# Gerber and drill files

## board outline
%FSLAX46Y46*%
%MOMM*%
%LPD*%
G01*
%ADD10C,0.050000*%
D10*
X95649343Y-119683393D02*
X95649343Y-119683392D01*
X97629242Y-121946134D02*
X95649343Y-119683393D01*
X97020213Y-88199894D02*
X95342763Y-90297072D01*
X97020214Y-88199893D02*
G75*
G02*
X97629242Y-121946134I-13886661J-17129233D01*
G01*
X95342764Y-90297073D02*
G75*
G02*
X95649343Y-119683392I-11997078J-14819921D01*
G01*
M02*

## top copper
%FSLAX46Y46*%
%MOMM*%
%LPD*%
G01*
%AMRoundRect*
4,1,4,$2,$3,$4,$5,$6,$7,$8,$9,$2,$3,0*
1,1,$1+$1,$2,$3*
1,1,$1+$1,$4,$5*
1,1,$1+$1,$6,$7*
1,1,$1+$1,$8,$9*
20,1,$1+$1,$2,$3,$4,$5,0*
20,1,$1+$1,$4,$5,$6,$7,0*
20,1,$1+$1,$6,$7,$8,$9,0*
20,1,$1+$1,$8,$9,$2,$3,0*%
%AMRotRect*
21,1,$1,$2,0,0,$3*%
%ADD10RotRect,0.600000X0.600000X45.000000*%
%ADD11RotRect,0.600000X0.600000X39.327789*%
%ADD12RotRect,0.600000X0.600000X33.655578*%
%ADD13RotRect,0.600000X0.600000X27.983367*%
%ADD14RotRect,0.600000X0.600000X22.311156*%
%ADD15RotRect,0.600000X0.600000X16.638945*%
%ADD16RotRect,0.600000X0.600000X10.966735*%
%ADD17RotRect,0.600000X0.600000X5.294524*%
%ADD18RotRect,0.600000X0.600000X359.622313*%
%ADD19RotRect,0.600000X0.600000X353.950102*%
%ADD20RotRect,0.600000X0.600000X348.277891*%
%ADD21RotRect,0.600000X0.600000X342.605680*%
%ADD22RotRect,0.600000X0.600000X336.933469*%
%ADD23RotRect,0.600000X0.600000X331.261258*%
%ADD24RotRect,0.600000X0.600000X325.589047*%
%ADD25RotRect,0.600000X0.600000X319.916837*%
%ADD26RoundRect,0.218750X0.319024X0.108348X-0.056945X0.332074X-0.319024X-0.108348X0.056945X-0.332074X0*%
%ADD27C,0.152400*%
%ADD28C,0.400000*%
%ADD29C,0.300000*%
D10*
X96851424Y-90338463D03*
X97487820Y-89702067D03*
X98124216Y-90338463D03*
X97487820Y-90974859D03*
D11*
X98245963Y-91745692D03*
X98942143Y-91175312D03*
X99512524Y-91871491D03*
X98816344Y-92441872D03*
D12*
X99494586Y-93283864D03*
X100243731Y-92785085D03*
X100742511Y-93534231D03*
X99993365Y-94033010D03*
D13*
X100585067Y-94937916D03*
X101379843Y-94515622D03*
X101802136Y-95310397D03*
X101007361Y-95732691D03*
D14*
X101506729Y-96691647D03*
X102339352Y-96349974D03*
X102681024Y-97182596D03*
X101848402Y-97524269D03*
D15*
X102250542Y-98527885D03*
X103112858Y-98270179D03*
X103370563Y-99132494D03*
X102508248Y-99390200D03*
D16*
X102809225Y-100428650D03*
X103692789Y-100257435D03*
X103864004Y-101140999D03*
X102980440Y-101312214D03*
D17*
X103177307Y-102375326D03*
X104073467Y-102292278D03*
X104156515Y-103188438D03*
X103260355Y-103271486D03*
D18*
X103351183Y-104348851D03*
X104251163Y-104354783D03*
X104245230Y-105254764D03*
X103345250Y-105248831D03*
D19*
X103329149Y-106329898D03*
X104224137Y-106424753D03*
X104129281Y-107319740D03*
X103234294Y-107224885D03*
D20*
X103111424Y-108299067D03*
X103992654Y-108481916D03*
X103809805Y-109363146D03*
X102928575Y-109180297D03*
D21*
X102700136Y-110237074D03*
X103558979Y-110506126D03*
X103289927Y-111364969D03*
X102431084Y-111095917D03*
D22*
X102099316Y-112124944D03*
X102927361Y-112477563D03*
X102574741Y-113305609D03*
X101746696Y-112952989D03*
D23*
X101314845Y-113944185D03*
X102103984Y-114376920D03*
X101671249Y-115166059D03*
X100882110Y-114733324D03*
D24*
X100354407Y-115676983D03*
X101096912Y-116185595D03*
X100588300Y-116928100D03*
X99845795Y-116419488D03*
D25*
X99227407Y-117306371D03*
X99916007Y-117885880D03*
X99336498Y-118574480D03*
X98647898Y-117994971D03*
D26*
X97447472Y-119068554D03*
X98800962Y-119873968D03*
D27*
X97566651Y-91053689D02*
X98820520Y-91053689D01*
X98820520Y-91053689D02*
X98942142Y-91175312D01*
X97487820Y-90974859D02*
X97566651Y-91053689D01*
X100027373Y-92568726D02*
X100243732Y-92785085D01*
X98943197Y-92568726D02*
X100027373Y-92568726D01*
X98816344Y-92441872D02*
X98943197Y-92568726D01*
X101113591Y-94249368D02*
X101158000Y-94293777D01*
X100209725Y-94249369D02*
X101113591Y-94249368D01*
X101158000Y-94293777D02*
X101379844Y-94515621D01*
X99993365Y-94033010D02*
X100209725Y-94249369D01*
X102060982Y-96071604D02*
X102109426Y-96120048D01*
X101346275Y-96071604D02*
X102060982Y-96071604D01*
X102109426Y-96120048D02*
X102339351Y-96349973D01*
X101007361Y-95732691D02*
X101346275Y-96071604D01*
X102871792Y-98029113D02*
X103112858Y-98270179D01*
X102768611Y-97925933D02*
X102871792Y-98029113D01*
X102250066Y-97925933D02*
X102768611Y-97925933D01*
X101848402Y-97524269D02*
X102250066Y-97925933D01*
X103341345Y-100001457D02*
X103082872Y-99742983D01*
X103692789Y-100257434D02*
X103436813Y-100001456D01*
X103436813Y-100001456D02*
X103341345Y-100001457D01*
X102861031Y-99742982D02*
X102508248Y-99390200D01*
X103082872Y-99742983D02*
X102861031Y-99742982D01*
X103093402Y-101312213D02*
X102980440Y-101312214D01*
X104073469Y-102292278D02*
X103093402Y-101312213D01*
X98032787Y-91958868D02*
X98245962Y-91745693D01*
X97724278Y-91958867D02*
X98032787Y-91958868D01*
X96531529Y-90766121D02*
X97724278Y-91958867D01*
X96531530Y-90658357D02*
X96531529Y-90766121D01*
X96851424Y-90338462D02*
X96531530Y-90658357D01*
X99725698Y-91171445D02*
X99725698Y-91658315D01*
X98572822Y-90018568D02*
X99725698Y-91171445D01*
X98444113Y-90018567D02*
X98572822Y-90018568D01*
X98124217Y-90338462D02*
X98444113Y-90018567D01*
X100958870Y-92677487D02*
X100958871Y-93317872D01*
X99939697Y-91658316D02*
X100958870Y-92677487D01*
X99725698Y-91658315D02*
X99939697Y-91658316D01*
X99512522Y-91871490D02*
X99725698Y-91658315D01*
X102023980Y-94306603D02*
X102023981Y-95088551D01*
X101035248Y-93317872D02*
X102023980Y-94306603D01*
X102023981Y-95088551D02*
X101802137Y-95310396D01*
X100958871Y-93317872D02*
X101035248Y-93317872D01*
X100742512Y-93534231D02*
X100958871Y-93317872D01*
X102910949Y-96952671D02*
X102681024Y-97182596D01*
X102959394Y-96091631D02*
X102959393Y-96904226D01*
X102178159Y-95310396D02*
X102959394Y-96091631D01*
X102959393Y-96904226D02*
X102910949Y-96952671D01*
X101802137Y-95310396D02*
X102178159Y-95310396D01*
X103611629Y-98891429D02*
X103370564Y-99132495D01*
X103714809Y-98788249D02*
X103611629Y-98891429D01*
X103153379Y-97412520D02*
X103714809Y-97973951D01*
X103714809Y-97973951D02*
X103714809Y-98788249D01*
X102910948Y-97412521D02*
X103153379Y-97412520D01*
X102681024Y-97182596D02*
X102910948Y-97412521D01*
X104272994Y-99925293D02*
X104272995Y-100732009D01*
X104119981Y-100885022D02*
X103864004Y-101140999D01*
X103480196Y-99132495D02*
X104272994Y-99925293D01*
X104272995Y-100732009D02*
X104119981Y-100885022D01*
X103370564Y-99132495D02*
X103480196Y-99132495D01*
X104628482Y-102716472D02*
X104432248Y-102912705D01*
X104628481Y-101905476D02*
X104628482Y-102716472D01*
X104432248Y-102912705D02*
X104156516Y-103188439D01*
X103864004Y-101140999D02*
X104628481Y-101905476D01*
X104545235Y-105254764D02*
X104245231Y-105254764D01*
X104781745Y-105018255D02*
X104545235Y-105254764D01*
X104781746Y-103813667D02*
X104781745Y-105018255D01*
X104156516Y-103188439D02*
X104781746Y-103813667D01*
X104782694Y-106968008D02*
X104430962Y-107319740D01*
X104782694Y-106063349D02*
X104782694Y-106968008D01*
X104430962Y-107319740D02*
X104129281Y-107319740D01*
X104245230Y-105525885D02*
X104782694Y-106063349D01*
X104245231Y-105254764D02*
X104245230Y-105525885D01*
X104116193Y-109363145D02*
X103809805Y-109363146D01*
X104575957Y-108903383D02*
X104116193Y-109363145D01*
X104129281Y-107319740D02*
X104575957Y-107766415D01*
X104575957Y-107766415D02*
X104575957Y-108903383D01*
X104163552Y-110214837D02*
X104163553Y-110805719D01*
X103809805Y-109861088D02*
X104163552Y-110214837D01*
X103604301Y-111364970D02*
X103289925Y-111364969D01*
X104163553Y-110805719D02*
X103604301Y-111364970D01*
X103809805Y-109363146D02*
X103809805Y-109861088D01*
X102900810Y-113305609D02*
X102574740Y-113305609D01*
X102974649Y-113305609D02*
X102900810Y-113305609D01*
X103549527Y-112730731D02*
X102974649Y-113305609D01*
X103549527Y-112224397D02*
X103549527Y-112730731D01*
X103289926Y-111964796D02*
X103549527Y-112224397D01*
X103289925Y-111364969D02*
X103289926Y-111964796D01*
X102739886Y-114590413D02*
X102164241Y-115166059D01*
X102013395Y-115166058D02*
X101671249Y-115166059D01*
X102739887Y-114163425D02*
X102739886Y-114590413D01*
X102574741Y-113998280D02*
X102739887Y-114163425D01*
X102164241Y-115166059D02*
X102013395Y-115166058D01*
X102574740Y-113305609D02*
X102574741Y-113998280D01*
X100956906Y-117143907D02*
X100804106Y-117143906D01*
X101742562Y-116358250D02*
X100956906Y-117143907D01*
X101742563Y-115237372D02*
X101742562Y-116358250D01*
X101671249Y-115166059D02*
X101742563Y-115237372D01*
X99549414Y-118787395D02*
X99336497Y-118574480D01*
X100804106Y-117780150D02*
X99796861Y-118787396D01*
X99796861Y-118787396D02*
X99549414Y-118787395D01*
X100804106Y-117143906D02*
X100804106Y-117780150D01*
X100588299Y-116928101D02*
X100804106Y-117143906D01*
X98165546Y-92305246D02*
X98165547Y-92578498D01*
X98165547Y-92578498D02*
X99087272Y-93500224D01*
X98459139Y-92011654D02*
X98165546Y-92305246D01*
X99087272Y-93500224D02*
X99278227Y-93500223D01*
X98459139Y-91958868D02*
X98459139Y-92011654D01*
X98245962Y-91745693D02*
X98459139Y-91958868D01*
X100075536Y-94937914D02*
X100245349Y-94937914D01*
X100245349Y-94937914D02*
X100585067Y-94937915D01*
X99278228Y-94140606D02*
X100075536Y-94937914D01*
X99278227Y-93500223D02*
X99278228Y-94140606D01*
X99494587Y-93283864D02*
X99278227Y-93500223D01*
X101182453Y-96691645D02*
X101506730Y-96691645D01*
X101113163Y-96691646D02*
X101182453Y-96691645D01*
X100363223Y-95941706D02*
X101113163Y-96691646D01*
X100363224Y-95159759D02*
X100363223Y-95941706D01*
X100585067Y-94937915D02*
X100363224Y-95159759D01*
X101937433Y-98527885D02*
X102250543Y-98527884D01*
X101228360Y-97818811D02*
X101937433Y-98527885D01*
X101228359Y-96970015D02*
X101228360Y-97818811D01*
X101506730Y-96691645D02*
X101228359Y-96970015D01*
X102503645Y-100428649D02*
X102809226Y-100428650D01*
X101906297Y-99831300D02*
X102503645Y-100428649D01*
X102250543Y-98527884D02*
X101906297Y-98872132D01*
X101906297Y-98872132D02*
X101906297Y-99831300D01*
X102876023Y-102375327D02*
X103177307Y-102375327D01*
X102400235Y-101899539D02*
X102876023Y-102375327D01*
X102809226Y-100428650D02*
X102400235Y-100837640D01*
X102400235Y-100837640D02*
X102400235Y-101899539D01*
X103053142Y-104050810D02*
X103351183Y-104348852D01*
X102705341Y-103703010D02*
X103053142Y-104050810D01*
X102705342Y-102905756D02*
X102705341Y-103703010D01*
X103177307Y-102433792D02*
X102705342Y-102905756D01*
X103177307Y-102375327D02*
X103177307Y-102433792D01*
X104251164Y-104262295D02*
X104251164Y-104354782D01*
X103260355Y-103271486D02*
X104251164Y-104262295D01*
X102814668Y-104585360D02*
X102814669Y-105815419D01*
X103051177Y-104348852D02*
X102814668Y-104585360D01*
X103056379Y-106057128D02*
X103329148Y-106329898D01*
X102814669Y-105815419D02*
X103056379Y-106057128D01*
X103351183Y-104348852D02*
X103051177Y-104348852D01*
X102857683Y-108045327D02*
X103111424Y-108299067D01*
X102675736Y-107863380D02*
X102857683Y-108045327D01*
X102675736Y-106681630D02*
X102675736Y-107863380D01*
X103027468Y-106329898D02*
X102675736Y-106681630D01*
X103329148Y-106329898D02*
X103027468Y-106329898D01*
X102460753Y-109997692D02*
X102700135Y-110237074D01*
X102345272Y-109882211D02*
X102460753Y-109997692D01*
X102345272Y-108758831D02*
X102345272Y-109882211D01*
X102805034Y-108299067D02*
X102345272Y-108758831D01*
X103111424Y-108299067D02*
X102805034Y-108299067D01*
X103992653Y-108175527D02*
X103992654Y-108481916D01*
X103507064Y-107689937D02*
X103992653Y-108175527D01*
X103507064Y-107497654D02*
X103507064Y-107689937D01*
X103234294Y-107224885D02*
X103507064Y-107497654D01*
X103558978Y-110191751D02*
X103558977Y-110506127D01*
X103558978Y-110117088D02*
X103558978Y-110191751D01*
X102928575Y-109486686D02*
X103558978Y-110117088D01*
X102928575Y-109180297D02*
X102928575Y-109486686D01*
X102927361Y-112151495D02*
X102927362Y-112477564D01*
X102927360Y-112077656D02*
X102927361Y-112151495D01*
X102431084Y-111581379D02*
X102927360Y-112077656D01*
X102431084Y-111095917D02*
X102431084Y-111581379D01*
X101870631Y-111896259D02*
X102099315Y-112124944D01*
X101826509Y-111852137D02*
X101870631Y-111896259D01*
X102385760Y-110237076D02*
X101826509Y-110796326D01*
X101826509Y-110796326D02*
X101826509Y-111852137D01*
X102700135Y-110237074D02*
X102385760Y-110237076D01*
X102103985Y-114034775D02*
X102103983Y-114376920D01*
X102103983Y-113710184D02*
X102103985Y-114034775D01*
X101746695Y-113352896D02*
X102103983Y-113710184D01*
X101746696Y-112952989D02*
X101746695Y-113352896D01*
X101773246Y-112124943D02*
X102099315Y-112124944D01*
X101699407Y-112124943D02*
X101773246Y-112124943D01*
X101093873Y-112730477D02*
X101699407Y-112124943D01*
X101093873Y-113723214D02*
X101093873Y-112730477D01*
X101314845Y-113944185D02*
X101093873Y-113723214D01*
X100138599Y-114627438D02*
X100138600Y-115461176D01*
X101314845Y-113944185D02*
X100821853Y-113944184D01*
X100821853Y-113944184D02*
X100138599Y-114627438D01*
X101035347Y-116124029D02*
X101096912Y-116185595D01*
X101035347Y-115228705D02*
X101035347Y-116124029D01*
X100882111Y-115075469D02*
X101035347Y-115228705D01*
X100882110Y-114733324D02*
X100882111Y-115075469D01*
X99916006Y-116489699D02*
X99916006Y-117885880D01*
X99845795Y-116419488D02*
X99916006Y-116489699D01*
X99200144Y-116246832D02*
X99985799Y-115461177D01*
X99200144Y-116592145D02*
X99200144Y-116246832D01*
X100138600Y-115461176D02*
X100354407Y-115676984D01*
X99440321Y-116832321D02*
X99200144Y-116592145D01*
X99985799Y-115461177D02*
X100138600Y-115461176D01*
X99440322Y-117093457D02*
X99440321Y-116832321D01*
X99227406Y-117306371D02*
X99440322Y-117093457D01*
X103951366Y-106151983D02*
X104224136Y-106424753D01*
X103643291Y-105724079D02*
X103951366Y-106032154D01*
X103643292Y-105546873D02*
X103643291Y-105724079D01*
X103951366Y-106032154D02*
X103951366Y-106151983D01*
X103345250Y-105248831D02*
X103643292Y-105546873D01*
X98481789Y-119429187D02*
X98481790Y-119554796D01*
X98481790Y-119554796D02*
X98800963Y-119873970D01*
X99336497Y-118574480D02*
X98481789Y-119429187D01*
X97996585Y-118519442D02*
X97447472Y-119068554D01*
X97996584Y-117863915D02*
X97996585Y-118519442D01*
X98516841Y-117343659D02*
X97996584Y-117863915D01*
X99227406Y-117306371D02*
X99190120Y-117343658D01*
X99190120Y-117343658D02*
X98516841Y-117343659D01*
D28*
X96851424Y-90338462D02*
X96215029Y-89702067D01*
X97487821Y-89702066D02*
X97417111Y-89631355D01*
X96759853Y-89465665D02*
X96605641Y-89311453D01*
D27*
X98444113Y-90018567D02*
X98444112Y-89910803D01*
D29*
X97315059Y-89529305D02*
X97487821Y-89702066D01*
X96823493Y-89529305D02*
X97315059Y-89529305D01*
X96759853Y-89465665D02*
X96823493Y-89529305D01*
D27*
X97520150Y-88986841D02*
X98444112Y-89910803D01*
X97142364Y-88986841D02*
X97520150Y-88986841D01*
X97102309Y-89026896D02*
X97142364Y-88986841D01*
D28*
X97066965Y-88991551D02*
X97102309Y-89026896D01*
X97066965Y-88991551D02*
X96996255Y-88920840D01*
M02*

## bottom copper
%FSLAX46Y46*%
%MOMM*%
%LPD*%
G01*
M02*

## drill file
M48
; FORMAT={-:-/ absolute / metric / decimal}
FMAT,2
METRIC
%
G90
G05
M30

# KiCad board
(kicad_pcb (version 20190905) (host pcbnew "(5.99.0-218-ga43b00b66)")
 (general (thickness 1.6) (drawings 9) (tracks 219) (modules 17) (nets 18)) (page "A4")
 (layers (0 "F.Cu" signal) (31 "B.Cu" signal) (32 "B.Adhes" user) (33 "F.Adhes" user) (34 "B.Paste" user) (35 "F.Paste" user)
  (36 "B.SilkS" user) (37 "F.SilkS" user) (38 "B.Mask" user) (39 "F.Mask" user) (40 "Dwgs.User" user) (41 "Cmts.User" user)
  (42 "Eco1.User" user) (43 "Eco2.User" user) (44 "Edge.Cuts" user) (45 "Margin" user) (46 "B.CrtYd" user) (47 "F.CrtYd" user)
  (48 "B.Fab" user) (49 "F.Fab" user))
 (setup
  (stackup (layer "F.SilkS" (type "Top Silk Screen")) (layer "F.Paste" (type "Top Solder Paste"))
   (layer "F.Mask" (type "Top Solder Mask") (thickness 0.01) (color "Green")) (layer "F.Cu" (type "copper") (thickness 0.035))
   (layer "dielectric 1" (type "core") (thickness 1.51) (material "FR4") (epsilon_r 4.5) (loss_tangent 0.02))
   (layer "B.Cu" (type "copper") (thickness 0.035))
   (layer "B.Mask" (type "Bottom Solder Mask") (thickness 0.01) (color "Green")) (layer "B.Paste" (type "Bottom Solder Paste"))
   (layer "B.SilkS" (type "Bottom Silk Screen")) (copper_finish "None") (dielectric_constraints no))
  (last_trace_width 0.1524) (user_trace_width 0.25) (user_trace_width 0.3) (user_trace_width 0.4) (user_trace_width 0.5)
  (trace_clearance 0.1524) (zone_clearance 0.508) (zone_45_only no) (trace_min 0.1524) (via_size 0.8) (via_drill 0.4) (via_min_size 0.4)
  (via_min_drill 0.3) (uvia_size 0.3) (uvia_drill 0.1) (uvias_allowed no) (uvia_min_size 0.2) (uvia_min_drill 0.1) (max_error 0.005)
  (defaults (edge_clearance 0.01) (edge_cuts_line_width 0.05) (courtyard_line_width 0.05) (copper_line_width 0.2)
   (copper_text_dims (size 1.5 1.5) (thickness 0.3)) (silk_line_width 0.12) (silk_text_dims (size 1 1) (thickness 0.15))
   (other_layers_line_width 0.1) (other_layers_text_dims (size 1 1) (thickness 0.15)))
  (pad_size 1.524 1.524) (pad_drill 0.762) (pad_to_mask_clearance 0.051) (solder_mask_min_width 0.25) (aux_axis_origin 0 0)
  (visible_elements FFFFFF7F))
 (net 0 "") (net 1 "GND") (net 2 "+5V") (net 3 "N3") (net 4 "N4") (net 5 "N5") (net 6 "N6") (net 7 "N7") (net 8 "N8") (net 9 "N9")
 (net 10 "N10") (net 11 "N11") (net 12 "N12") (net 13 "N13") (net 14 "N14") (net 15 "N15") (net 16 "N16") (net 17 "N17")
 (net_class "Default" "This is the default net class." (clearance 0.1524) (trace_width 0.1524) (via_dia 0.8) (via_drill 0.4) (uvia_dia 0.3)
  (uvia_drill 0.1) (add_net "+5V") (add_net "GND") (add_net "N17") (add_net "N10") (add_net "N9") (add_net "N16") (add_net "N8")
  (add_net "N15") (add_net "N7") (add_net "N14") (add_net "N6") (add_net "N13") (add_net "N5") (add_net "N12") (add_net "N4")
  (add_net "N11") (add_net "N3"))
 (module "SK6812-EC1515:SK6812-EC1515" (layer "F.Cu") (at 97.48782 90.974859 45)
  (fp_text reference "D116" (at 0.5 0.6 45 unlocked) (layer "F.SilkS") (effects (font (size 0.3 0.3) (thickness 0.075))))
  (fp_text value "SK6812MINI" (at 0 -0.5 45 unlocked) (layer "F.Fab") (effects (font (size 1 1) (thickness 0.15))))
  (pad "4" smd rect (at 0 -0.9 45) (size 0.6 0.6) (layers "F.Cu" "F.Paste" "F.Mask") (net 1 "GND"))
  (pad "3" smd rect (at 0.9 -0.9 45) (size 0.6 0.6) (layers "F.Cu" "F.Paste" "F.Mask"))
  (pad "2" smd rect (at 0.9 0 45) (size 0.6 0.6) (layers "F.Cu" "F.Paste" "F.Mask") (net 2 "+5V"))
  (pad "1" smd rect (at 0 0 45) (size 0.6 0.6) (layers "F.Cu" "F.Paste" "F.Mask") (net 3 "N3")))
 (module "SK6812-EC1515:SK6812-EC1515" (layer "F.Cu") (at 98.816344 92.441872 39.32778911)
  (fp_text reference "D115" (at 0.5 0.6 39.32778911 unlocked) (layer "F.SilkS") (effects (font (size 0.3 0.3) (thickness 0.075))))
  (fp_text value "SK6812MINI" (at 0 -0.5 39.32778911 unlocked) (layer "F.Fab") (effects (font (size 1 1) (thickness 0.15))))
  (pad "4" smd rect (at 0 -0.9 39.3277891) (size 0.6 0.6) (layers "F.Cu" "F.Paste" "F.Mask") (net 1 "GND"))
  (pad "3" smd rect (at 0.9 -0.9 39.3277891) (size 0.6 0.6) (layers "F.Cu" "F.Paste" "F.Mask") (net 3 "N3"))
  (pad "2" smd rect (at 0.9 0 39.3277891) (size 0.6 0.6) (layers "F.Cu" "F.Paste" "F.Mask") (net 2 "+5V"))
  (pad "1" smd rect (at 0 0 39.3277891) (size 0.6 0.6) (layers "F.Cu" "F.Paste" "F.Mask") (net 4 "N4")))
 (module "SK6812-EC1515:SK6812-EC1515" (layer "F.Cu") (at 99.993365 94.03301 33.65557821)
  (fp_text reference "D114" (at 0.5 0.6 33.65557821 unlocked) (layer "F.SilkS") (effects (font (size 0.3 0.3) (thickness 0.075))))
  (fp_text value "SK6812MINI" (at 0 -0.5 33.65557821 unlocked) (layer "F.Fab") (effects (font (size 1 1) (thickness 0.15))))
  (pad "4" smd rect (at 0 -0.9 33.6555782) (size 0.6 0.6) (layers "F.Cu" "F.Paste" "F.Mask") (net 1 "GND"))
  (pad "3" smd rect (at 0.9 -0.9 33.6555782) (size 0.6 0.6) (layers "F.Cu" "F.Paste" "F.Mask") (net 4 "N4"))
  (pad "2" smd rect (at 0.9 0 33.6555782) (size 0.6 0.6) (layers "F.Cu" "F.Paste" "F.Mask") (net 2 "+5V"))
  (pad "1" smd rect (at 0 0 33.6555782) (size 0.6 0.6) (layers "F.Cu" "F.Paste" "F.Mask") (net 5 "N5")))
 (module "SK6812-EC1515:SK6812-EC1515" (layer "F.Cu") (at 101.007361 95.732691 27.98336732)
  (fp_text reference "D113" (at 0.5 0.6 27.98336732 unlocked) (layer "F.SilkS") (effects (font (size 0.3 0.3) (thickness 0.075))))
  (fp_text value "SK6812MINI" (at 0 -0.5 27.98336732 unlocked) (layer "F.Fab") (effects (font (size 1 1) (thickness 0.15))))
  (pad "4" smd rect (at 0 -0.9 27.9833673) (size 0.6 0.6) (layers "F.Cu" "F.Paste" "F.Mask") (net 1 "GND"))
  (pad "3" smd rect (at 0.9 -0.9 27.9833673) (size 0.6 0.6) (layers "F.Cu" "F.Paste" "F.Mask") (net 5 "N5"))
  (pad "2" smd rect (at 0.9 0 27.9833673) (size 0.6 0.6) (layers "F.Cu" "F.Paste" "F.Mask") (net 2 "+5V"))
  (pad "1" smd rect (at 0 0 27.9833673) (size 0.6 0.6) (layers "F.Cu" "F.Paste" "F.Mask") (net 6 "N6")))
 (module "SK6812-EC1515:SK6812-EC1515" (layer "F.Cu") (at 101.848402 97.524269 22.31115642)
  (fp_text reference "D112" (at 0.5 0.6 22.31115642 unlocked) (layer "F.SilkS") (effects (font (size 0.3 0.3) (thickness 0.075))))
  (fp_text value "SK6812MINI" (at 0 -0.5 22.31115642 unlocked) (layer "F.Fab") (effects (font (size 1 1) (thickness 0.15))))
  (pad "4" smd rect (at 0 -0.9 22.3111564) (size 0.6 0.6) (layers "F.Cu" "F.Paste" "F.Mask") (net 1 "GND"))
  (pad "3" smd rect (at 0.9 -0.9 22.3111564) (size 0.6 0.6) (layers "F.Cu" "F.Paste" "F.Mask") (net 6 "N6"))
  (pad "2" smd rect (at 0.9 0 22.3111564) (size 0.6 0.6) (layers "F.Cu" "F.Paste" "F.Mask") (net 2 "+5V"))
  (pad "1" smd rect (at 0 0 22.3111564) (size 0.6 0.6) (layers "F.Cu" "F.Paste" "F.Mask") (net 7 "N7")))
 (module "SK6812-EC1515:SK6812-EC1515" (layer "F.Cu") (at 102.508248 99.3902 16.63894553)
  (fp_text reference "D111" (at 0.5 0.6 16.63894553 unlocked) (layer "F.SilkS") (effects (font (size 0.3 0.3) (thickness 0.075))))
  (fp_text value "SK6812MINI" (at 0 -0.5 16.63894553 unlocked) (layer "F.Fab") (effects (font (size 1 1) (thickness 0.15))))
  (pad "4" smd rect (at 0 -0.9 16.6389455) (size 0.6 0.6) (layers "F.Cu" "F.Paste" "F.Mask") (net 1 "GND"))
  (pad "3" smd rect (at 0.9 -0.9 16.6389455) (size 0.6 0.6) (layers "F.Cu" "F.Paste" "F.Mask") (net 7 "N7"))
  (pad "2" smd rect (at 0.9 0 16.6389455) (size 0.6 0.6) (layers "F.Cu" "F.Paste" "F.Mask") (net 2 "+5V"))
  (pad "1" smd rect (at 0 0 16.6389455) (size 0.6 0.6) (layers "F.Cu" "F.Paste" "F.Mask") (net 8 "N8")))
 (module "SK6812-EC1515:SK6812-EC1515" (layer "F.Cu") (at 102.98044 101.312214 10.96673463)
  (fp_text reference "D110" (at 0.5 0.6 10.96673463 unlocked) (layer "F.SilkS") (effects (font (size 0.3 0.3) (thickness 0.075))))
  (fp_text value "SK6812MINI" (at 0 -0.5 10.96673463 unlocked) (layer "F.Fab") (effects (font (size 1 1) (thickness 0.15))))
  (pad "4" smd rect (at 0 -0.9 10.9667346) (size 0.6 0.6) (layers "F.Cu" "F.Paste" "F.Mask") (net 1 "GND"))
  (pad "3" smd rect (at 0.9 -0.9 10.9667346) (size 0.6 0.6) (layers "F.Cu" "F.Paste" "F.Mask") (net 8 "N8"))
  (pad "2" smd rect (at 0.9 0 10.9667346) (size 0.6 0.6) (layers "F.Cu" "F.Paste" "F.Mask") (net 2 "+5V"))
  (pad "1" smd rect (at 0 0 10.9667346) (size 0.6 0.6) (layers "F.Cu" "F.Paste" "F.Mask") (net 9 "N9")))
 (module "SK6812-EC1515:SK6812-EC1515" (layer "F.Cu") (at 103.260355 103.271486 5.29452374)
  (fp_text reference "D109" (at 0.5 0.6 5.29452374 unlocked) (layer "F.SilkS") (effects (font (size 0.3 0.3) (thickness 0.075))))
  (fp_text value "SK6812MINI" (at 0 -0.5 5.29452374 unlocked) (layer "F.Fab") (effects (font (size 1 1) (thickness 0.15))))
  (pad "4" smd rect (at 0 -0.9 5.2945237) (size 0.6 0.6) (layers "F.Cu" "F.Paste" "F.Mask") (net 1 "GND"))
  (pad "3" smd rect (at 0.9 -0.9 5.2945237) (size 0.6 0.6) (layers "F.Cu" "F.Paste" "F.Mask") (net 9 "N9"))
  (pad "2" smd rect (at 0.9 0 5.2945237) (size 0.6 0.6) (layers "F.Cu" "F.Paste" "F.Mask") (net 2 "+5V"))
  (pad "1" smd rect (at 0 0 5.2945237) (size 0.6 0.6) (layers "F.Cu" "F.Paste" "F.Mask") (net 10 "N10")))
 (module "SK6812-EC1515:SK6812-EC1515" (layer "F.Cu") (at 103.34525 105.248831 -0.37768716)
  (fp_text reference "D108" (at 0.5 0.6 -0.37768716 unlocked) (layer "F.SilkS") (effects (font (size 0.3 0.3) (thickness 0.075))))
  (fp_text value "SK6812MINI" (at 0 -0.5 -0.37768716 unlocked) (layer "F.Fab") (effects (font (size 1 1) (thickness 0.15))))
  (pad "4" smd rect (at 0 -0.9 359.6223128) (size 0.6 0.6) (layers "F.Cu" "F.Paste" "F.Mask") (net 1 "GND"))
  (pad "3" smd rect (at 0.9 -0.9 359.6223128) (size 0.6 0.6) (layers "F.Cu" "F.Paste" "F.Mask") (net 10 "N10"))
  (pad "2" smd rect (at 0.9 0 359.6223128) (size 0.6 0.6) (layers "F.Cu" "F.Paste" "F.Mask") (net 2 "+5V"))
  (pad "1" smd rect (at 0 0 359.6223128) (size 0.6 0.6) (layers "F.Cu" "F.Paste" "F.Mask") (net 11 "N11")))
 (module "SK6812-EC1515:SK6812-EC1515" (layer "F.Cu") (at 103.234294 107.224885 -6.04989805)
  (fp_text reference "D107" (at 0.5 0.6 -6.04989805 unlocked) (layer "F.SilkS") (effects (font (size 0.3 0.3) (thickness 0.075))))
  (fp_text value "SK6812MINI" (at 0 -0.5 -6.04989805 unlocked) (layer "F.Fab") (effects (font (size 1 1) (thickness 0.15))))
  (pad "4" smd rect (at 0 -0.9 353.9501019) (size 0.6 0.6) (layers "F.Cu" "F.Paste" "F.Mask") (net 1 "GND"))
  (pad "3" smd rect (at 0.9 -0.9 353.9501019) (size 0.6 0.6) (layers "F.Cu" "F.Paste" "F.Mask") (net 11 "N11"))
  (pad "2" smd rect (at 0.9 0 353.9501019) (size 0.6 0.6) (layers "F.Cu" "F.Paste" "F.Mask") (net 2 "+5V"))
  (pad "1" smd rect (at 0 0 353.9501019) (size 0.6 0.6) (layers "F.Cu" "F.Paste" "F.Mask") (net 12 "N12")))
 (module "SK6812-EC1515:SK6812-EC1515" (layer "F.Cu") (at 102.928575 109.180297 -11.72210895)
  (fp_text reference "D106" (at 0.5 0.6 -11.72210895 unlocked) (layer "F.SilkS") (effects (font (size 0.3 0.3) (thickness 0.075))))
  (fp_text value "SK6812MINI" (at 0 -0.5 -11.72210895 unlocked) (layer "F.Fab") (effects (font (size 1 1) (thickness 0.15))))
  (pad "4" smd rect (at 0 -0.9 348.2778911) (size 0.6 0.6) (layers "F.Cu" "F.Paste" "F.Mask") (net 1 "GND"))
  (pad "3" smd rect (at 0.9 -0.9 348.2778911) (size 0.6 0.6) (layers "F.Cu" "F.Paste" "F.Mask") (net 12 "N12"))
  (pad "2" smd rect (at 0.9 0 348.2778911) (size 0.6 0.6) (layers "F.Cu" "F.Paste" "F.Mask") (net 2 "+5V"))
  (pad "1" smd rect (at 0 0 348.2778911) (size 0.6 0.6) (layers "F.Cu" "F.Paste" "F.Mask") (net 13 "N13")))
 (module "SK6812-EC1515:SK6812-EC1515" (layer "F.Cu") (at 102.431084 111.095917 -17.39431984)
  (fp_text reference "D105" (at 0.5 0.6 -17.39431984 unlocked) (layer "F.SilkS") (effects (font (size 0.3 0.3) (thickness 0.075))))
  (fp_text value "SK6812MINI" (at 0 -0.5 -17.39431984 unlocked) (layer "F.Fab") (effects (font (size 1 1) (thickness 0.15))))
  (pad "4" smd rect (at 0 -0.9 342.6056802) (size 0.6 0.6) (layers "F.Cu" "F.Paste" "F.Mask") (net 1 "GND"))
  (pad "3" smd rect (at 0.9 -0.9 342.6056802) (size 0.6 0.6) (layers "F.Cu" "F.Paste" "F.Mask") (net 13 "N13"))
  (pad "2" smd rect (at 0.9 0 342.6056802) (size 0.6 0.6) (layers "F.Cu" "F.Paste" "F.Mask") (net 2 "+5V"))
  (pad "1" smd rect (at 0 0 342.6056802) (size 0.6 0.6) (layers "F.Cu" "F.Paste" "F.Mask") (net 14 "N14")))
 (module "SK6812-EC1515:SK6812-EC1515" (layer "F.Cu") (at 101.746696 112.952989 -23.06653074)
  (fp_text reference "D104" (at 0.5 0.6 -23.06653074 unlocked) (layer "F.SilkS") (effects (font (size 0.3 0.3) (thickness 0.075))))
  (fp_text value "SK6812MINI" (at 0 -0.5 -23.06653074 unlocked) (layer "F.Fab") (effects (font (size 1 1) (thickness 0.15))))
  (pad "4" smd rect (at 0 -0.9 336.9334693) (size 0.6 0.6) (layers "F.Cu" "F.Paste" "F.Mask") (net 1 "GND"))
  (pad "3" smd rect (at 0.9 -0.9 336.9334693) (size 0.6 0.6) (layers "F.Cu" "F.Paste" "F.Mask") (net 14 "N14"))
  (pad "2" smd rect (at 0.9 0 336.9334693) (size 0.6 0.6) (layers "F.Cu" "F.Paste" "F.Mask") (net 2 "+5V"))
  (pad "1" smd rect (at 0 0 336.9334693) (size 0.6 0.6) (layers "F.Cu" "F.Paste" "F.Mask") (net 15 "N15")))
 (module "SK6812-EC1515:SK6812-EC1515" (layer "F.Cu") (at 100.88211 114.733324 -28.73874163)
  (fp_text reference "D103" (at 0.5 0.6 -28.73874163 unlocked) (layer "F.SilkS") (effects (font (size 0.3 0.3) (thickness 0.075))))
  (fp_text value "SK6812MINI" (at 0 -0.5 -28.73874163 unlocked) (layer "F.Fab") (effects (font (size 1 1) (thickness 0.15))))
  (pad "4" smd rect (at 0 -0.9 331.2612584) (size 0.6 0.6) (layers "F.Cu" "F.Paste" "F.Mask") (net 1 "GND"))
  (pad "3" smd rect (at 0.9 -0.9 331.2612584) (size 0.6 0.6) (layers "F.Cu" "F.Paste" "F.Mask") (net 15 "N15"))
  (pad "2" smd rect (at 0.9 0 331.2612584) (size 0.6 0.6) (layers "F.Cu" "F.Paste" "F.Mask") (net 2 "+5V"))
  (pad "1" smd rect (at 0 0 331.2612584) (size 0.6 0.6) (layers "F.Cu" "F.Paste" "F.Mask") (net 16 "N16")))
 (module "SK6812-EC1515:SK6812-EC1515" (layer "F.Cu") (at 99.845795 116.419488 -34.41095253)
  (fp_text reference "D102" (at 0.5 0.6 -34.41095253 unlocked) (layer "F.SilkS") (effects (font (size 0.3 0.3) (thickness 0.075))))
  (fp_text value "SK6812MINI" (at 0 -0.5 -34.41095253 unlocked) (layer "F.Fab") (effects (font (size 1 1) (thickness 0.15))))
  (pad "4" smd rect (at 0 -0.9 325.5890475) (size 0.6 0.6) (layers "F.Cu" "F.Paste" "F.Mask") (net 1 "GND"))
  (pad "3" smd rect (at 0.9 -0.9 325.5890475) (size 0.6 0.6) (layers "F.Cu" "F.Paste" "F.Mask") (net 16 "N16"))
  (pad "2" smd rect (at 0.9 0 325.5890475) (size 0.6 0.6) (layers "F.Cu" "F.Paste" "F.Mask") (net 2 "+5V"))
  (pad "1" smd rect (at 0 0 325.5890475) (size 0.6 0.6) (layers "F.Cu" "F.Paste" "F.Mask") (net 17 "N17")))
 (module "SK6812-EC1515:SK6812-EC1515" (layer "F.Cu") (at 98.647898 117.994971 -40.08316342)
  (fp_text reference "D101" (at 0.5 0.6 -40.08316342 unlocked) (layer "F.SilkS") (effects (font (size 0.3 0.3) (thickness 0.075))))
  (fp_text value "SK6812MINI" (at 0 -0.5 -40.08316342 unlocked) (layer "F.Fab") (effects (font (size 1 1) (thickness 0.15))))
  (pad "4" smd rect (at 0 -0.9 319.9168366) (size 0.6 0.6) (layers "F.Cu" "F.Paste" "F.Mask") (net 1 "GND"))
  (pad "3" smd rect (at 0.9 -0.9 319.9168366) (size 0.6 0.6) (layers "F.Cu" "F.Paste" "F.Mask") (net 17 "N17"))
  (pad "2" smd rect (at 0.9 0 319.9168366) (size 0.6 0.6) (layers "F.Cu" "F.Paste" "F.Mask") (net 2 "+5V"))
  (pad "1" smd rect (at 0 0 319.9168366) (size 0.6 0.6) (layers "F.Cu" "F.Paste" "F.Mask")))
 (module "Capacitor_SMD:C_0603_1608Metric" (layer "F.Cu") (at 98.124217 119.471261 149.2446257)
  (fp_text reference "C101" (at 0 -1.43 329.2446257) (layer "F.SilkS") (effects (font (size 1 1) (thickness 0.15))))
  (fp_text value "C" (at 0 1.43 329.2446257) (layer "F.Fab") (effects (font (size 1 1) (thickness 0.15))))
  (pad "2" smd roundrect (at 0.7875 0 149.2446257) (size 0.875 0.95) (layers "F.Cu" "F.Paste" "F.Mask") (roundrect_rratio 0.25)
   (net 1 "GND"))
  (pad "1" smd roundrect (at -0.7875 0 149.2446257) (size 0.875 0.95) (layers "F.Cu" "F.Paste" "F.Mask") (roundrect_rratio 0.25)
   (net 2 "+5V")))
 (gr_line (start 95.649343 119.683393) (end 95.649343 119.683392) (layer "Edge.Cuts") (width 0.05))
 (gr_line (start 97.629242 121.946134) (end 95.649343 119.683393) (layer "Edge.Cuts") (width 0.05))
 (gr_line (start 97.020213 88.199894) (end 95.342763 90.297072) (layer "Edge.Cuts") (width 0.05))
 (gr_arc (start 83.133553 105.329126) (end 97.629242 121.946134) (angle -99.86882594) (layer "Edge.Cuts") (width 0.05))
 (gr_arc (start 83.345686 105.116994) (end 95.649343 119.683392) (angle -100.8225569) (layer "Edge.Cuts") (width 0.05))
 (segment (start 97.566651 91.053689) (end 98.82052 91.053689) (width 0.1524) (layer "F.Cu") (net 3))
 (segment (start 98.82052 91.053689) (end 98.942142 91.175312) (width 0.1524) (layer "F.Cu") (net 3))
 (segment (start 97.48782 90.974859) (end 97.566651 91.053689) (width 0.1524) (layer "F.Cu") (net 3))
 (segment (start 100.027373 92.568726) (end 100.243732 92.785085) (width 0.1524) (layer "F.Cu") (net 4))
 (segment (start 98.943197 92.568726) (end 100.027373 92.568726) (width 0.1524) (layer "F.Cu") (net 4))
 (segment (start 98.816344 92.441872) (end 98.943197 92.568726) (width 0.1524) (layer "F.Cu") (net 4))
 (segment (start 101.113591 94.249368) (end 101.158 94.293777) (width 0.1524) (layer "F.Cu") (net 5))
 (segment (start 100.209725 94.249369) (end 101.113591 94.249368) (width 0.1524) (layer "F.Cu") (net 5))
 (segment (start 101.158 94.293777) (end 101.379844 94.515621) (width 0.1524) (layer "F.Cu") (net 5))
 (segment (start 99.993365 94.03301) (end 100.209725 94.249369) (width 0.1524) (layer "F.Cu") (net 5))
 (segment (start 102.060982 96.071604) (end 102.109426 96.120048) (width 0.1524) (layer "F.Cu") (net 6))
 (segment (start 101.346275 96.071604) (end 102.060982 96.071604) (width 0.1524) (layer "F.Cu") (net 6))
 (segment (start 102.109426 96.120048) (end 102.339351 96.349973) (width 0.1524) (layer "F.Cu") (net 6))
 (segment (start 101.007361 95.732691) (end 101.346275 96.071604) (width 0.1524) (layer "F.Cu") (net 6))
 (segment (start 102.871792 98.029113) (end 103.112858 98.270179) (width 0.1524) (layer "F.Cu") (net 7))
 (segment (start 102.768611 97.925933) (end 102.871792 98.029113) (width 0.1524) (layer "F.Cu") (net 7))
 (segment (start 102.250066 97.925933) (end 102.768611 97.925933) (width 0.1524) (layer "F.Cu") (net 7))
 (segment (start 101.848402 97.524269) (end 102.250066 97.925933) (width 0.1524) (layer "F.Cu") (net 7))
 (segment (start 103.341345 100.001457) (end 103.082872 99.742983) (width 0.1524) (layer "F.Cu") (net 8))
 (segment (start 103.692789 100.257434) (end 103.436813 100.001456) (width 0.1524) (layer "F.Cu") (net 8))
 (segment (start 103.436813 100.001456) (end 103.341345 100.001457) (width 0.1524) (layer "F.Cu") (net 8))
 (segment (start 102.861031 99.742982) (end 102.508248 99.3902) (width 0.1524) (layer "F.Cu") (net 8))
 (segment (start 103.082872 99.742983) (end 102.861031 99.742982) (width 0.1524) (layer "F.Cu") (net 8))
 (segment (start 103.093402 101.312213) (end 102.98044 101.312214) (width 0.1524) (layer "F.Cu") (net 9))
 (segment (start 104.073469 102.292278) (end 103.093402 101.312213) (width 0.1524) (layer "F.Cu") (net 9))
 (segment (start 98.032787 91.958868) (end 98.245962 91.745693) (width 0.1524) (layer "F.Cu") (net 1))
 (segment (start 97.724278 91.958867) (end 98.032787 91.958868) (width 0.1524) (layer "F.Cu") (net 1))
 (segment (start 96.531529 90.766121) (end 97.724278 91.958867) (width 0.1524) (layer "F.Cu") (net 1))
 (segment (start 96.53153 90.658357) (end 96.531529 90.766121) (width 0.1524) (layer "F.Cu") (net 1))
 (segment (start 96.851424 90.338462) (end 96.53153 90.658357) (width 0.1524) (layer "F.Cu") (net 1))
 (segment (start 99.725698 91.171445) (end 99.725698 91.658315) (width 0.1524) (layer "F.Cu") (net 2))
 (segment (start 98.572822 90.018568) (end 99.725698 91.171445) (width 0.1524) (layer "F.Cu") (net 2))
 (segment (start 98.444113 90.018567) (end 98.572822 90.018568) (width 0.1524) (layer "F.Cu") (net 2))
 (segment (start 98.124217 90.338462) (end 98.444113 90.018567) (width 0.1524) (layer "F.Cu") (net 2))
 (segment (start 100.95887 92.677487) (end 100.958871 93.317872) (width 0.1524) (layer "F.Cu") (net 2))
 (segment (start 99.939697 91.658316) (end 100.95887 92.677487) (width 0.1524) (layer "F.Cu") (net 2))
 (segment (start 99.725698 91.658315) (end 99.939697 91.658316) (width 0.1524) (layer "F.Cu") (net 2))
 (segment (start 99.512522 91.87149) (end 99.725698 91.658315) (width 0.1524) (layer "F.Cu") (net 2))
 (segment (start 102.02398 94.306603) (end 102.023981 95.088551) (width 0.1524) (layer "F.Cu") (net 2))
 (segment (start 101.035248 93.317872) (end 102.02398 94.306603) (width 0.1524) (layer "F.Cu") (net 2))
 (segment (start 102.023981 95.088551) (end 101.802137 95.310396) (width 0.1524) (layer "F.Cu") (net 2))
 (segment (start 100.958871 93.317872) (end 101.035248 93.317872) (width 0.1524) (layer "F.Cu") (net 2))
 (segment (start 100.742512 93.534231) (end 100.958871 93.317872) (width 0.1524) (layer "F.Cu") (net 2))
 (segment (start 102.910949 96.952671) (end 102.681024 97.182596) (width 0.1524) (layer "F.Cu") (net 2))
 (segment (start 102.959394 96.091631) (end 102.959393 96.904226) (width 0.1524) (layer "F.Cu") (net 2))
 (segment (start 102.178159 95.310396) (end 102.959394 96.091631) (width 0.1524) (layer "F.Cu") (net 2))
 (segment (start 102.959393 96.904226) (end 102.910949 96.952671) (width 0.1524) (layer "F.Cu") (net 2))
 (segment (start 101.802137 95.310396) (end 102.178159 95.310396) (width 0.1524) (layer "F.Cu") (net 2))
 (segment (start 103.611629 98.891429) (end 103.370564 99.132495) (width 0.1524) (layer "F.Cu") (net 2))
 (segment (start 103.714809 98.788249) (end 103.611629 98.891429) (width 0.1524) (layer "F.Cu") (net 2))
 (segment (start 103.153379 97.41252) (end 103.714809 97.973951) (width 0.1524) (layer "F.Cu") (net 2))
 (segment (start 103.714809 97.973951) (end 103.714809 98.788249) (width 0.1524) (layer "F.Cu") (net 2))
 (segment (start 102.910948 97.412521) (end 103.153379 97.41252) (width 0.1524) (layer "F.Cu") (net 2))
 (segment (start 102.681024 97.182596) (end 102.910948 97.412521) (width 0.1524) (layer "F.Cu") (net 2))
 (segment (start 104.272994 99.925293) (end 104.272995 100.732009) (width 0.1524) (layer "F.Cu") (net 2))
 (segment (start 104.119981 100.885022) (end 103.864004 101.140999) (width 0.1524) (layer "F.Cu") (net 2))
 (segment (start 103.480196 99.132495) (end 104.272994 99.925293) (width 0.1524) (layer "F.Cu") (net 2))
 (segment (start 104.272995 100.732009) (end 104.119981 100.885022) (width 0.1524) (layer "F.Cu") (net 2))
 (segment (start 103.370564 99.132495) (end 103.480196 99.132495) (width 0.1524) (layer "F.Cu") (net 2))
 (segment (start 104.628482 102.716472) (end 104.432248 102.912705) (width 0.1524) (layer "F.Cu") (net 2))
 (segment (start 104.628481 101.905476) (end 104.628482 102.716472) (width 0.1524) (layer "F.Cu") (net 2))
 (segment (start 104.432248 102.912705) (end 104.156516 103.188439) (width 0.1524) (layer "F.Cu") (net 2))
 (segment (start 103.864004 101.140999) (end 104.628481 101.905476) (width 0.1524) (layer "F.Cu") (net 2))
 (segment (start 104.545235 105.254764) (end 104.245231 105.254764) (width 0.1524) (layer "F.Cu") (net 2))
 (segment (start 104.781745 105.018255) (end 104.545235 105.254764) (width 0.1524) (layer "F.Cu") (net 2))
 (segment (start 104.781746 103.813667) (end 104.781745 105.018255) (width 0.1524) (layer "F.Cu") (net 2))
 (segment (start 104.156516 103.188439) (end 104.781746 103.813667) (width 0.1524) (layer "F.Cu") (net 2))
 (segment (start 104.782694 106.968008) (end 104.430962 107.31974) (width 0.1524) (layer "F.Cu") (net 2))
 (segment (start 104.782694 106.063349) (end 104.782694 106.968008) (width 0.1524) (layer "F.Cu") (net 2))
 (segment (start 104.430962 107.31974) (end 104.129281 107.31974) (width 0.1524) (layer "F.Cu") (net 2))
 (segment (start 104.24523 105.525885) (end 104.782694 106.063349) (width 0.1524) (layer "F.Cu") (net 2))
 (segment (start 104.245231 105.254764) (end 104.24523 105.525885) (width 0.1524) (layer "F.Cu") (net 2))
 (segment (start 104.116193 109.363145) (end 103.809805 109.363146) (width 0.1524) (layer "F.Cu") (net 2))
 (segment (start 104.575957 108.903383) (end 104.116193 109.363145) (width 0.1524) (layer "F.Cu") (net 2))
 (segment (start 104.129281 107.31974) (end 104.575957 107.766415) (width 0.1524) (layer "F.Cu") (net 2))
 (segment (start 104.575957 107.766415) (end 104.575957 108.903383) (width 0.1524) (layer "F.Cu") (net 2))
 (segment (start 104.163552 110.214837) (end 104.163553 110.805719) (width 0.1524) (layer "F.Cu") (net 2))
 (segment (start 103.809805 109.861088) (end 104.163552 110.214837) (width 0.1524) (layer "F.Cu") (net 2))
 (segment (start 103.604301 111.36497) (end 103.289925 111.364969) (width 0.1524) (layer "F.Cu") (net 2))
 (segment (start 104.163553 110.805719) (end 103.604301 111.36497) (width 0.1524) (layer "F.Cu") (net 2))
 (segment (start 103.809805 109.363146) (end 103.809805 109.861088) (width 0.1524) (layer "F.Cu") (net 2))
 (segment (start 102.90081 113.305609) (end 102.57474 113.305609) (width 0.1524) (layer "F.Cu") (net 2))
 (segment (start 102.974649 113.305609) (end 102.90081 113.305609) (width 0.1524) (layer "F.Cu") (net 2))
 (segment (start 103.549527 112.730731) (end 102.974649 113.305609) (width 0.1524) (layer "F.Cu") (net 2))
 (segment (start 103.549527 112.224397) (end 103.549527 112.730731) (width 0.1524) (layer "F.Cu") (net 2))
 (segment (start 103.289926 111.964796) (end 103.549527 112.224397) (width 0.1524) (layer "F.Cu") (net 2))
 (segment (start 103.289925 111.364969) (end 103.289926 111.964796) (width 0.1524) (layer "F.Cu") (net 2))
 (segment (start 102.739886 114.590413) (end 102.164241 115.166059) (width 0.1524) (layer "F.Cu") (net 2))
 (segment (start 102.013395 115.166058) (end 101.671249 115.166059) (width 0.1524) (layer "F.Cu") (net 2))
 (segment (start 102.739887 114.163425) (end 102.739886 114.590413) (width 0.1524) (layer "F.Cu") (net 2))
 (segment (start 102.574741 113.99828) (end 102.739887 114.163425) (width 0.1524) (layer "F.Cu") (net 2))
 (segment (start 102.164241 115.166059) (end 102.013395 115.166058) (width 0.1524) (layer "F.Cu") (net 2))
 (segment (start 102.57474 113.305609) (end 102.574741 113.99828) (width 0.1524) (layer "F.Cu") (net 2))
 (segment (start 100.956906 117.143907) (end 100.804106 117.143906) (width 0.1524) (layer "F.Cu") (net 2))
 (segment (start 101.742562 116.35825) (end 100.956906 117.143907) (width 0.1524) (layer "F.Cu") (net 2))
 (segment (start 101.742563 115.237372) (end 101.742562 116.35825) (width 0.1524) (layer "F.Cu") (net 2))
 (segment (start 101.671249 115.166059) (end 101.742563 115.237372) (width 0.1524) (layer "F.Cu") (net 2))
 (segment (start 99.549414 118.787395) (end 99.336497 118.57448) (width 0.1524) (layer "F.Cu") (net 2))
 (segment (start 100.804106 117.78015) (end 99.796861 118.787396) (width 0.1524) (layer "F.Cu") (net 2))
 (segment (start 99.796861 118.787396) (end 99.549414 118.787395) (width 0.1524) (layer "F.Cu") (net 2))
 (segment (start 100.804106 117.143906) (end 100.804106 117.78015) (width 0.1524) (layer "F.Cu") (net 2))
 (segment (start 100.588299 116.928101) (end 100.804106 117.143906) (width 0.1524) (layer "F.Cu") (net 2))
 (segment (start 98.165546 92.305246) (end 98.165547 92.578498) (width 0.1524) (layer "F.Cu") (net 1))
 (segment (start 98.165547 92.578498) (end 99.087272 93.500224) (width 0.1524) (layer "F.Cu") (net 1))
 (segment (start 98.459139 92.011654) (end 98.165546 92.305246) (width 0.1524) (layer "F.Cu") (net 1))
 (segment (start 99.087272 93.500224) (end 99.278227 93.500223) (width 0.1524) (layer "F.Cu") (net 1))
 (segment (start 98.459139 91.958868) (end 98.459139 92.011654) (width 0.1524) (layer "F.Cu") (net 1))
 (segment (start 98.245962 91.745693) (end 98.459139 91.958868) (width 0.1524) (layer "F.Cu") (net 1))
 (segment (start 100.075536 94.937914) (end 100.245349 94.937914) (width 0.1524) (layer "F.Cu") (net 1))
 (segment (start 100.245349 94.937914) (end 100.585067 94.937915) (width 0.1524) (layer "F.Cu") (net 1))
 (segment (start 99.278228 94.140606) (end 100.075536 94.937914) (width 0.1524) (layer "F.Cu") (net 1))
 (segment (start 99.278227 93.500223) (end 99.278228 94.140606) (width 0.1524) (layer "F.Cu") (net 1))
 (segment (start 99.494587 93.283864) (end 99.278227 93.500223) (width 0.1524) (layer "F.Cu") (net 1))
 (segment (start 101.182453 96.691645) (end 101.50673 96.691645) (width 0.1524) (layer "F.Cu") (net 1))
 (segment (start 101.113163 96.691646) (end 101.182453 96.691645) (width 0.1524) (layer "F.Cu") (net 1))
 (segment (start 100.363223 95.941706) (end 101.113163 96.691646) (width 0.1524) (layer "F.Cu") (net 1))
 (segment (start 100.363224 95.159759) (end 100.363223 95.941706) (width 0.1524) (layer "F.Cu") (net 1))
 (segment (start 100.585067 94.937915) (end 100.363224 95.159759) (width 0.1524) (layer "F.Cu") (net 1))
 (segment (start 101.937433 98.527885) (end 102.250543 98.527884) (width 0.1524) (layer "F.Cu") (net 1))
 (segment (start 101.22836 97.818811) (end 101.937433 98.527885) (width 0.1524) (layer "F.Cu") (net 1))
 (segment (start 101.228359 96.970015) (end 101.22836 97.818811) (width 0.1524) (layer "F.Cu") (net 1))
 (segment (start 101.50673 96.691645) (end 101.228359 96.970015) (width 0.1524) (layer "F.Cu") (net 1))
 (segment (start 102.503645 100.428649) (end 102.809226 100.42865) (width 0.1524) (layer "F.Cu") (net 1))
 (segment (start 101.906297 99.8313) (end 102.503645 100.428649) (width 0.1524) (layer "F.Cu") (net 1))
 (segment (start 102.250543 98.527884) (end 101.906297 98.872132) (width 0.1524) (layer "F.Cu") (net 1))
 (segment (start 101.906297 98.872132) (end 101.906297 99.8313) (width 0.1524) (layer "F.Cu") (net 1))
 (segment (start 102.876023 102.375327) (end 103.177307 102.375327) (width 0.1524) (layer "F.Cu") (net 1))
 (segment (start 102.400235 101.899539) (end 102.876023 102.375327) (width 0.1524) (layer "F.Cu") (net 1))
 (segment (start 102.809226 100.42865) (end 102.400235 100.83764) (width 0.1524) (layer "F.Cu") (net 1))
 (segment (start 102.400235 100.83764) (end 102.400235 101.899539) (width 0.1524) (layer "F.Cu") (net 1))
 (segment (start 103.053142 104.05081) (end 103.351183 104.348852) (width 0.1524) (layer "F.Cu") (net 1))
 (segment (start 102.705341 103.70301) (end 103.053142 104.05081) (width 0.1524) (layer "F.Cu") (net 1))
 (segment (start 102.705342 102.905756) (end 102.705341 103.70301) (width 0.1524) (layer "F.Cu") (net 1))
 (segment (start 103.177307 102.433792) (end 102.705342 102.905756) (width 0.1524) (layer "F.Cu") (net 1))
 (segment (start 103.177307 102.375327) (end 103.177307 102.433792) (width 0.1524) (layer "F.Cu") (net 1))
 (segment (start 104.251164 104.262295) (end 104.251164 104.354782) (width 0.1524) (layer "F.Cu") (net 10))
 (segment (start 103.260355 103.271486) (end 104.251164 104.262295) (width 0.1524) (layer "F.Cu") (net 10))
 (segment (start 102.814668 104.58536) (end 102.814669 105.815419) (width 0.1524) (layer "F.Cu") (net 1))
 (segment (start 103.051177 104.348852) (end 102.814668 104.58536) (width 0.1524) (layer "F.Cu") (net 1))
 (segment (start 103.056379 106.057128) (end 103.329148 106.329898) (width 0.1524) (layer "F.Cu") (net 1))
 (segment (start 102.814669 105.815419) (end 103.056379 106.057128) (width 0.1524) (layer "F.Cu") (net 1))
 (segment (start 103.351183 104.348852) (end 103.051177 104.348852) (width 0.1524) (layer "F.Cu") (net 1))
 (segment (start 102.857683 108.045327) (end 103.111424 108.299067) (width 0.1524) (layer "F.Cu") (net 1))
 (segment (start 102.675736 107.86338) (end 102.857683 108.045327) (width 0.1524) (layer "F.Cu") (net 1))
 (segment (start 102.675736 106.68163) (end 102.675736 107.86338) (width 0.1524) (layer "F.Cu") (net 1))
 (segment (start 103.027468 106.329898) (end 102.675736 106.68163) (width 0.1524) (layer "F.Cu") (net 1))
 (segment (start 103.329148 106.329898) (end 103.027468 106.329898) (width 0.1524) (layer "F.Cu") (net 1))
 (segment (start 102.460753 109.997692) (end 102.700135 110.237074) (width 0.1524) (layer "F.Cu") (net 1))
 (segment (start 102.345272 109.882211) (end 102.460753 109.997692) (width 0.1524) (layer "F.Cu") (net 1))
 (segment (start 102.345272 108.758831) (end 102.345272 109.882211) (width 0.1524) (layer "F.Cu") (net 1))
 (segment (start 102.805034 108.299067) (end 102.345272 108.758831) (width 0.1524) (layer "F.Cu") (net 1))
 (segment (start 103.111424 108.299067) (end 102.805034 108.299067) (width 0.1524) (layer "F.Cu") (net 1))
 (segment (start 103.992653 108.175527) (end 103.992654 108.481916) (width 0.1524) (layer "F.Cu") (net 12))
 (segment (start 103.507064 107.689937) (end 103.992653 108.175527) (width 0.1524) (layer "F.Cu") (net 12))
 (segment (start 103.507064 107.497654) (end 103.507064 107.689937) (width 0.1524) (layer "F.Cu") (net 12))
 (segment (start 103.234294 107.224885) (end 103.507064 107.497654) (width 0.1524) (layer "F.Cu") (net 12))
 (segment (start 103.558978 110.191751) (end 103.558977 110.506127) (width 0.1524) (layer "F.Cu") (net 13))
 (segment (start 103.558978 110.117088) (end 103.558978 110.191751) (width 0.1524) (layer "F.Cu") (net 13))
 (segment (start 102.928575 109.486686) (end 103.558978 110.117088) (width 0.1524) (layer "F.Cu") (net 13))
 (segment (start 102.928575 109.180297) (end 102.928575 109.486686) (width 0.1524) (layer "F.Cu") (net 13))
 (segment (start 102.927361 112.151495) (end 102.927362 112.477564) (width 0.1524) (layer "F.Cu") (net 14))
 (segment (start 102.92736 112.077656) (end 102.927361 112.151495) (width 0.1524) (layer "F.Cu") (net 14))
 (segment (start 102.431084 111.581379) (end 102.92736 112.077656) (width 0.1524) (layer "F.Cu") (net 14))
 (segment (start 102.431084 111.095917) (end 102.431084 111.581379) (width 0.1524) (layer "F.Cu") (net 14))
 (segment (start 101.870631 111.896259) (end 102.099315 112.124944) (width 0.1524) (layer "F.Cu") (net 1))
 (segment (start 101.826509 111.852137) (end 101.870631 111.896259) (width 0.1524) (layer "F.Cu") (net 1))
 (segment (start 102.38576 110.237076) (end 101.826509 110.796326) (width 0.1524) (layer "F.Cu") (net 1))
 (segment (start 101.826509 110.796326) (end 101.826509 111.852137) (width 0.1524) (layer "F.Cu") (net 1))
 (segment (start 102.700135 110.237074) (end 102.38576 110.237076) (width 0.1524) (layer "F.Cu") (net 1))
 (segment (start 102.103985 114.034775) (end 102.103983 114.37692) (width 0.1524) (layer "F.Cu") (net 15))
 (segment (start 102.103983 113.710184) (end 102.103985 114.034775) (width 0.1524) (layer "F.Cu") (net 15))
 (segment (start 101.746695 113.352896) (end 102.103983 113.710184) (width 0.1524) (layer "F.Cu") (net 15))
 (segment (start 101.746696 112.952989) (end 101.746695 113.352896) (width 0.1524) (layer "F.Cu") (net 15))
 (segment (start 101.773246 112.124943) (end 102.099315 112.124944) (width 0.1524) (layer "F.Cu") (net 1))
 (segment (start 101.699407 112.124943) (end 101.773246 112.124943) (width 0.1524) (layer "F.Cu") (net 1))
 (segment (start 101.093873 112.730477) (end 101.699407 112.124943) (width 0.1524) (layer "F.Cu") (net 1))
 (segment (start 101.093873 113.723214) (end 101.093873 112.730477) (width 0.1524) (layer "F.Cu") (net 1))
 (segment (start 101.314845 113.944185) (end 101.093873 113.723214) (width 0.1524) (layer "F.Cu") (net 1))
 (segment (start 100.138599 114.627438) (end 100.1386 115.461176) (width 0.1524) (layer "F.Cu") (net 1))
 (segment (start 101.314845 113.944185) (end 100.821853 113.944184) (width 0.1524) (layer "F.Cu") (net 1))
 (segment (start 100.821853 113.944184) (end 100.138599 114.627438) (width 0.1524) (layer "F.Cu") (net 1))
 (segment (start 101.035347 116.124029) (end 101.096912 116.185595) (width 0.1524) (layer "F.Cu") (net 16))
 (segment (start 101.035347 115.228705) (end 101.035347 116.124029) (width 0.1524) (layer "F.Cu") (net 16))
 (segment (start 100.882111 115.075469) (end 101.035347 115.228705) (width 0.1524) (layer "F.Cu") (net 16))
 (segment (start 100.88211 114.733324) (end 100.882111 115.075469) (width 0.1524) (layer "F.Cu") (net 16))
 (segment (start 99.916006 116.489699) (end 99.916006 117.88588) (width 0.1524) (layer "F.Cu") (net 17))
 (segment (start 99.845795 116.419488) (end 99.916006 116.489699) (width 0.1524) (layer "F.Cu") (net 17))
 (segment (start 99.200144 116.246832) (end 99.985799 115.461177) (width 0.1524) (layer "F.Cu") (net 1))
 (segment (start 99.200144 116.592145) (end 99.200144 116.246832) (width 0.1524) (layer "F.Cu") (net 1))
 (segment (start 100.1386 115.461176) (end 100.354407 115.676984) (width 0.1524) (layer "F.Cu") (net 1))
 (segment (start 99.440321 116.832321) (end 99.200144 116.592145) (width 0.1524) (layer "F.Cu") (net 1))
 (segment (start 99.985799 115.461177) (end 100.1386 115.461176) (width 0.1524) (layer "F.Cu") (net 1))
 (segment (start 99.440322 117.093457) (end 99.440321 116.832321) (width 0.1524) (layer "F.Cu") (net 1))
 (segment (start 99.227406 117.306371) (end 99.440322 117.093457) (width 0.1524) (layer "F.Cu") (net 1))
 (segment (start 103.951366 106.151983) (end 104.224136 106.424753) (width 0.1524) (layer "F.Cu") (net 11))
 (segment (start 103.643291 105.724079) (end 103.951366 106.032154) (width 0.1524) (layer "F.Cu") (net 11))
 (segment (start 103.643292 105.546873) (end 103.643291 105.724079) (width 0.1524) (layer "F.Cu") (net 11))
 (segment (start 103.951366 106.032154) (end 103.951366 106.151983) (width 0.1524) (layer "F.Cu") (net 11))
 (segment (start 103.34525 105.248831) (end 103.643292 105.546873) (width 0.1524) (layer "F.Cu") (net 11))
 (segment (start 98.481789 119.429187) (end 98.48179 119.554796) (width 0.1524) (layer "F.Cu") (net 2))
 (segment (start 98.48179 119.554796) (end 98.800963 119.87397) (width 0.1524) (layer "F.Cu") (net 2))
 (segment (start 99.336497 118.57448) (end 98.481789 119.429187) (width 0.1524) (layer "F.Cu") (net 2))
 (segment (start 97.996585 118.519442) (end 97.447472 119.068554) (width 0.1524) (layer "F.Cu") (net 1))
 (segment (start 97.996584 117.863915) (end 97.996585 118.519442) (width 0.1524) (layer "F.Cu") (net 1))
 (segment (start 98.516841 117.343659) (end 97.996584 117.863915) (width 0.1524) (layer "F.Cu") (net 1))
 (segment (start 99.227406 117.306371) (end 99.19012 117.343658) (width 0.1524) (layer "F.Cu") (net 1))
 (segment (start 99.19012 117.343658) (end 98.516841 117.343659) (width 0.1524) (layer "F.Cu") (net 1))
 (segment (start 96.851424 90.338462) (end 96.215029 89.702067) (width 0.4) (layer "F.Cu") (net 1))
 (segment (start 97.487821 89.702066) (end 97.417111 89.631355) (width 0.4) (layer "F.Cu") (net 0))
 (segment (start 96.759853 89.465665) (end 96.605641 89.311453) (width 0.4) (layer "F.Cu") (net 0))
 (segment (start 98.444113 90.018567) (end 98.444112 89.910803) (width 0.1524) (layer "F.Cu") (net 2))
 (segment (start 97.315059 89.529305) (end 97.487821 89.702066) (width 0.3) (layer "F.Cu") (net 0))
 (segment (start 96.823493 89.529305) (end 97.315059 89.529305) (width 0.3) (layer "F.Cu") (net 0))
 (segment (start 96.759853 89.465665) (end 96.823493 89.529305) (width 0.3) (layer "F.Cu") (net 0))
 (segment (start 97.52015 88.986841) (end 98.444112 89.910803) (width 0.1524) (layer "F.Cu") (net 2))
 (segment (start 97.142364 88.986841) (end 97.52015 88.986841) (width 0.1524) (layer "F.Cu") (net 2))
 (segment (start 97.102309 89.026896) (end 97.142364 88.986841) (width 0.1524) (layer "F.Cu") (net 2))
 (segment (start 97.066965 88.991551) (end 97.102309 89.026896) (width 0.4) (layer "F.Cu") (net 2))
 (segment (start 97.066965 88.991551) (end 96.996255 88.92084) (width 0.4) (layer "F.Cu") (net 2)))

